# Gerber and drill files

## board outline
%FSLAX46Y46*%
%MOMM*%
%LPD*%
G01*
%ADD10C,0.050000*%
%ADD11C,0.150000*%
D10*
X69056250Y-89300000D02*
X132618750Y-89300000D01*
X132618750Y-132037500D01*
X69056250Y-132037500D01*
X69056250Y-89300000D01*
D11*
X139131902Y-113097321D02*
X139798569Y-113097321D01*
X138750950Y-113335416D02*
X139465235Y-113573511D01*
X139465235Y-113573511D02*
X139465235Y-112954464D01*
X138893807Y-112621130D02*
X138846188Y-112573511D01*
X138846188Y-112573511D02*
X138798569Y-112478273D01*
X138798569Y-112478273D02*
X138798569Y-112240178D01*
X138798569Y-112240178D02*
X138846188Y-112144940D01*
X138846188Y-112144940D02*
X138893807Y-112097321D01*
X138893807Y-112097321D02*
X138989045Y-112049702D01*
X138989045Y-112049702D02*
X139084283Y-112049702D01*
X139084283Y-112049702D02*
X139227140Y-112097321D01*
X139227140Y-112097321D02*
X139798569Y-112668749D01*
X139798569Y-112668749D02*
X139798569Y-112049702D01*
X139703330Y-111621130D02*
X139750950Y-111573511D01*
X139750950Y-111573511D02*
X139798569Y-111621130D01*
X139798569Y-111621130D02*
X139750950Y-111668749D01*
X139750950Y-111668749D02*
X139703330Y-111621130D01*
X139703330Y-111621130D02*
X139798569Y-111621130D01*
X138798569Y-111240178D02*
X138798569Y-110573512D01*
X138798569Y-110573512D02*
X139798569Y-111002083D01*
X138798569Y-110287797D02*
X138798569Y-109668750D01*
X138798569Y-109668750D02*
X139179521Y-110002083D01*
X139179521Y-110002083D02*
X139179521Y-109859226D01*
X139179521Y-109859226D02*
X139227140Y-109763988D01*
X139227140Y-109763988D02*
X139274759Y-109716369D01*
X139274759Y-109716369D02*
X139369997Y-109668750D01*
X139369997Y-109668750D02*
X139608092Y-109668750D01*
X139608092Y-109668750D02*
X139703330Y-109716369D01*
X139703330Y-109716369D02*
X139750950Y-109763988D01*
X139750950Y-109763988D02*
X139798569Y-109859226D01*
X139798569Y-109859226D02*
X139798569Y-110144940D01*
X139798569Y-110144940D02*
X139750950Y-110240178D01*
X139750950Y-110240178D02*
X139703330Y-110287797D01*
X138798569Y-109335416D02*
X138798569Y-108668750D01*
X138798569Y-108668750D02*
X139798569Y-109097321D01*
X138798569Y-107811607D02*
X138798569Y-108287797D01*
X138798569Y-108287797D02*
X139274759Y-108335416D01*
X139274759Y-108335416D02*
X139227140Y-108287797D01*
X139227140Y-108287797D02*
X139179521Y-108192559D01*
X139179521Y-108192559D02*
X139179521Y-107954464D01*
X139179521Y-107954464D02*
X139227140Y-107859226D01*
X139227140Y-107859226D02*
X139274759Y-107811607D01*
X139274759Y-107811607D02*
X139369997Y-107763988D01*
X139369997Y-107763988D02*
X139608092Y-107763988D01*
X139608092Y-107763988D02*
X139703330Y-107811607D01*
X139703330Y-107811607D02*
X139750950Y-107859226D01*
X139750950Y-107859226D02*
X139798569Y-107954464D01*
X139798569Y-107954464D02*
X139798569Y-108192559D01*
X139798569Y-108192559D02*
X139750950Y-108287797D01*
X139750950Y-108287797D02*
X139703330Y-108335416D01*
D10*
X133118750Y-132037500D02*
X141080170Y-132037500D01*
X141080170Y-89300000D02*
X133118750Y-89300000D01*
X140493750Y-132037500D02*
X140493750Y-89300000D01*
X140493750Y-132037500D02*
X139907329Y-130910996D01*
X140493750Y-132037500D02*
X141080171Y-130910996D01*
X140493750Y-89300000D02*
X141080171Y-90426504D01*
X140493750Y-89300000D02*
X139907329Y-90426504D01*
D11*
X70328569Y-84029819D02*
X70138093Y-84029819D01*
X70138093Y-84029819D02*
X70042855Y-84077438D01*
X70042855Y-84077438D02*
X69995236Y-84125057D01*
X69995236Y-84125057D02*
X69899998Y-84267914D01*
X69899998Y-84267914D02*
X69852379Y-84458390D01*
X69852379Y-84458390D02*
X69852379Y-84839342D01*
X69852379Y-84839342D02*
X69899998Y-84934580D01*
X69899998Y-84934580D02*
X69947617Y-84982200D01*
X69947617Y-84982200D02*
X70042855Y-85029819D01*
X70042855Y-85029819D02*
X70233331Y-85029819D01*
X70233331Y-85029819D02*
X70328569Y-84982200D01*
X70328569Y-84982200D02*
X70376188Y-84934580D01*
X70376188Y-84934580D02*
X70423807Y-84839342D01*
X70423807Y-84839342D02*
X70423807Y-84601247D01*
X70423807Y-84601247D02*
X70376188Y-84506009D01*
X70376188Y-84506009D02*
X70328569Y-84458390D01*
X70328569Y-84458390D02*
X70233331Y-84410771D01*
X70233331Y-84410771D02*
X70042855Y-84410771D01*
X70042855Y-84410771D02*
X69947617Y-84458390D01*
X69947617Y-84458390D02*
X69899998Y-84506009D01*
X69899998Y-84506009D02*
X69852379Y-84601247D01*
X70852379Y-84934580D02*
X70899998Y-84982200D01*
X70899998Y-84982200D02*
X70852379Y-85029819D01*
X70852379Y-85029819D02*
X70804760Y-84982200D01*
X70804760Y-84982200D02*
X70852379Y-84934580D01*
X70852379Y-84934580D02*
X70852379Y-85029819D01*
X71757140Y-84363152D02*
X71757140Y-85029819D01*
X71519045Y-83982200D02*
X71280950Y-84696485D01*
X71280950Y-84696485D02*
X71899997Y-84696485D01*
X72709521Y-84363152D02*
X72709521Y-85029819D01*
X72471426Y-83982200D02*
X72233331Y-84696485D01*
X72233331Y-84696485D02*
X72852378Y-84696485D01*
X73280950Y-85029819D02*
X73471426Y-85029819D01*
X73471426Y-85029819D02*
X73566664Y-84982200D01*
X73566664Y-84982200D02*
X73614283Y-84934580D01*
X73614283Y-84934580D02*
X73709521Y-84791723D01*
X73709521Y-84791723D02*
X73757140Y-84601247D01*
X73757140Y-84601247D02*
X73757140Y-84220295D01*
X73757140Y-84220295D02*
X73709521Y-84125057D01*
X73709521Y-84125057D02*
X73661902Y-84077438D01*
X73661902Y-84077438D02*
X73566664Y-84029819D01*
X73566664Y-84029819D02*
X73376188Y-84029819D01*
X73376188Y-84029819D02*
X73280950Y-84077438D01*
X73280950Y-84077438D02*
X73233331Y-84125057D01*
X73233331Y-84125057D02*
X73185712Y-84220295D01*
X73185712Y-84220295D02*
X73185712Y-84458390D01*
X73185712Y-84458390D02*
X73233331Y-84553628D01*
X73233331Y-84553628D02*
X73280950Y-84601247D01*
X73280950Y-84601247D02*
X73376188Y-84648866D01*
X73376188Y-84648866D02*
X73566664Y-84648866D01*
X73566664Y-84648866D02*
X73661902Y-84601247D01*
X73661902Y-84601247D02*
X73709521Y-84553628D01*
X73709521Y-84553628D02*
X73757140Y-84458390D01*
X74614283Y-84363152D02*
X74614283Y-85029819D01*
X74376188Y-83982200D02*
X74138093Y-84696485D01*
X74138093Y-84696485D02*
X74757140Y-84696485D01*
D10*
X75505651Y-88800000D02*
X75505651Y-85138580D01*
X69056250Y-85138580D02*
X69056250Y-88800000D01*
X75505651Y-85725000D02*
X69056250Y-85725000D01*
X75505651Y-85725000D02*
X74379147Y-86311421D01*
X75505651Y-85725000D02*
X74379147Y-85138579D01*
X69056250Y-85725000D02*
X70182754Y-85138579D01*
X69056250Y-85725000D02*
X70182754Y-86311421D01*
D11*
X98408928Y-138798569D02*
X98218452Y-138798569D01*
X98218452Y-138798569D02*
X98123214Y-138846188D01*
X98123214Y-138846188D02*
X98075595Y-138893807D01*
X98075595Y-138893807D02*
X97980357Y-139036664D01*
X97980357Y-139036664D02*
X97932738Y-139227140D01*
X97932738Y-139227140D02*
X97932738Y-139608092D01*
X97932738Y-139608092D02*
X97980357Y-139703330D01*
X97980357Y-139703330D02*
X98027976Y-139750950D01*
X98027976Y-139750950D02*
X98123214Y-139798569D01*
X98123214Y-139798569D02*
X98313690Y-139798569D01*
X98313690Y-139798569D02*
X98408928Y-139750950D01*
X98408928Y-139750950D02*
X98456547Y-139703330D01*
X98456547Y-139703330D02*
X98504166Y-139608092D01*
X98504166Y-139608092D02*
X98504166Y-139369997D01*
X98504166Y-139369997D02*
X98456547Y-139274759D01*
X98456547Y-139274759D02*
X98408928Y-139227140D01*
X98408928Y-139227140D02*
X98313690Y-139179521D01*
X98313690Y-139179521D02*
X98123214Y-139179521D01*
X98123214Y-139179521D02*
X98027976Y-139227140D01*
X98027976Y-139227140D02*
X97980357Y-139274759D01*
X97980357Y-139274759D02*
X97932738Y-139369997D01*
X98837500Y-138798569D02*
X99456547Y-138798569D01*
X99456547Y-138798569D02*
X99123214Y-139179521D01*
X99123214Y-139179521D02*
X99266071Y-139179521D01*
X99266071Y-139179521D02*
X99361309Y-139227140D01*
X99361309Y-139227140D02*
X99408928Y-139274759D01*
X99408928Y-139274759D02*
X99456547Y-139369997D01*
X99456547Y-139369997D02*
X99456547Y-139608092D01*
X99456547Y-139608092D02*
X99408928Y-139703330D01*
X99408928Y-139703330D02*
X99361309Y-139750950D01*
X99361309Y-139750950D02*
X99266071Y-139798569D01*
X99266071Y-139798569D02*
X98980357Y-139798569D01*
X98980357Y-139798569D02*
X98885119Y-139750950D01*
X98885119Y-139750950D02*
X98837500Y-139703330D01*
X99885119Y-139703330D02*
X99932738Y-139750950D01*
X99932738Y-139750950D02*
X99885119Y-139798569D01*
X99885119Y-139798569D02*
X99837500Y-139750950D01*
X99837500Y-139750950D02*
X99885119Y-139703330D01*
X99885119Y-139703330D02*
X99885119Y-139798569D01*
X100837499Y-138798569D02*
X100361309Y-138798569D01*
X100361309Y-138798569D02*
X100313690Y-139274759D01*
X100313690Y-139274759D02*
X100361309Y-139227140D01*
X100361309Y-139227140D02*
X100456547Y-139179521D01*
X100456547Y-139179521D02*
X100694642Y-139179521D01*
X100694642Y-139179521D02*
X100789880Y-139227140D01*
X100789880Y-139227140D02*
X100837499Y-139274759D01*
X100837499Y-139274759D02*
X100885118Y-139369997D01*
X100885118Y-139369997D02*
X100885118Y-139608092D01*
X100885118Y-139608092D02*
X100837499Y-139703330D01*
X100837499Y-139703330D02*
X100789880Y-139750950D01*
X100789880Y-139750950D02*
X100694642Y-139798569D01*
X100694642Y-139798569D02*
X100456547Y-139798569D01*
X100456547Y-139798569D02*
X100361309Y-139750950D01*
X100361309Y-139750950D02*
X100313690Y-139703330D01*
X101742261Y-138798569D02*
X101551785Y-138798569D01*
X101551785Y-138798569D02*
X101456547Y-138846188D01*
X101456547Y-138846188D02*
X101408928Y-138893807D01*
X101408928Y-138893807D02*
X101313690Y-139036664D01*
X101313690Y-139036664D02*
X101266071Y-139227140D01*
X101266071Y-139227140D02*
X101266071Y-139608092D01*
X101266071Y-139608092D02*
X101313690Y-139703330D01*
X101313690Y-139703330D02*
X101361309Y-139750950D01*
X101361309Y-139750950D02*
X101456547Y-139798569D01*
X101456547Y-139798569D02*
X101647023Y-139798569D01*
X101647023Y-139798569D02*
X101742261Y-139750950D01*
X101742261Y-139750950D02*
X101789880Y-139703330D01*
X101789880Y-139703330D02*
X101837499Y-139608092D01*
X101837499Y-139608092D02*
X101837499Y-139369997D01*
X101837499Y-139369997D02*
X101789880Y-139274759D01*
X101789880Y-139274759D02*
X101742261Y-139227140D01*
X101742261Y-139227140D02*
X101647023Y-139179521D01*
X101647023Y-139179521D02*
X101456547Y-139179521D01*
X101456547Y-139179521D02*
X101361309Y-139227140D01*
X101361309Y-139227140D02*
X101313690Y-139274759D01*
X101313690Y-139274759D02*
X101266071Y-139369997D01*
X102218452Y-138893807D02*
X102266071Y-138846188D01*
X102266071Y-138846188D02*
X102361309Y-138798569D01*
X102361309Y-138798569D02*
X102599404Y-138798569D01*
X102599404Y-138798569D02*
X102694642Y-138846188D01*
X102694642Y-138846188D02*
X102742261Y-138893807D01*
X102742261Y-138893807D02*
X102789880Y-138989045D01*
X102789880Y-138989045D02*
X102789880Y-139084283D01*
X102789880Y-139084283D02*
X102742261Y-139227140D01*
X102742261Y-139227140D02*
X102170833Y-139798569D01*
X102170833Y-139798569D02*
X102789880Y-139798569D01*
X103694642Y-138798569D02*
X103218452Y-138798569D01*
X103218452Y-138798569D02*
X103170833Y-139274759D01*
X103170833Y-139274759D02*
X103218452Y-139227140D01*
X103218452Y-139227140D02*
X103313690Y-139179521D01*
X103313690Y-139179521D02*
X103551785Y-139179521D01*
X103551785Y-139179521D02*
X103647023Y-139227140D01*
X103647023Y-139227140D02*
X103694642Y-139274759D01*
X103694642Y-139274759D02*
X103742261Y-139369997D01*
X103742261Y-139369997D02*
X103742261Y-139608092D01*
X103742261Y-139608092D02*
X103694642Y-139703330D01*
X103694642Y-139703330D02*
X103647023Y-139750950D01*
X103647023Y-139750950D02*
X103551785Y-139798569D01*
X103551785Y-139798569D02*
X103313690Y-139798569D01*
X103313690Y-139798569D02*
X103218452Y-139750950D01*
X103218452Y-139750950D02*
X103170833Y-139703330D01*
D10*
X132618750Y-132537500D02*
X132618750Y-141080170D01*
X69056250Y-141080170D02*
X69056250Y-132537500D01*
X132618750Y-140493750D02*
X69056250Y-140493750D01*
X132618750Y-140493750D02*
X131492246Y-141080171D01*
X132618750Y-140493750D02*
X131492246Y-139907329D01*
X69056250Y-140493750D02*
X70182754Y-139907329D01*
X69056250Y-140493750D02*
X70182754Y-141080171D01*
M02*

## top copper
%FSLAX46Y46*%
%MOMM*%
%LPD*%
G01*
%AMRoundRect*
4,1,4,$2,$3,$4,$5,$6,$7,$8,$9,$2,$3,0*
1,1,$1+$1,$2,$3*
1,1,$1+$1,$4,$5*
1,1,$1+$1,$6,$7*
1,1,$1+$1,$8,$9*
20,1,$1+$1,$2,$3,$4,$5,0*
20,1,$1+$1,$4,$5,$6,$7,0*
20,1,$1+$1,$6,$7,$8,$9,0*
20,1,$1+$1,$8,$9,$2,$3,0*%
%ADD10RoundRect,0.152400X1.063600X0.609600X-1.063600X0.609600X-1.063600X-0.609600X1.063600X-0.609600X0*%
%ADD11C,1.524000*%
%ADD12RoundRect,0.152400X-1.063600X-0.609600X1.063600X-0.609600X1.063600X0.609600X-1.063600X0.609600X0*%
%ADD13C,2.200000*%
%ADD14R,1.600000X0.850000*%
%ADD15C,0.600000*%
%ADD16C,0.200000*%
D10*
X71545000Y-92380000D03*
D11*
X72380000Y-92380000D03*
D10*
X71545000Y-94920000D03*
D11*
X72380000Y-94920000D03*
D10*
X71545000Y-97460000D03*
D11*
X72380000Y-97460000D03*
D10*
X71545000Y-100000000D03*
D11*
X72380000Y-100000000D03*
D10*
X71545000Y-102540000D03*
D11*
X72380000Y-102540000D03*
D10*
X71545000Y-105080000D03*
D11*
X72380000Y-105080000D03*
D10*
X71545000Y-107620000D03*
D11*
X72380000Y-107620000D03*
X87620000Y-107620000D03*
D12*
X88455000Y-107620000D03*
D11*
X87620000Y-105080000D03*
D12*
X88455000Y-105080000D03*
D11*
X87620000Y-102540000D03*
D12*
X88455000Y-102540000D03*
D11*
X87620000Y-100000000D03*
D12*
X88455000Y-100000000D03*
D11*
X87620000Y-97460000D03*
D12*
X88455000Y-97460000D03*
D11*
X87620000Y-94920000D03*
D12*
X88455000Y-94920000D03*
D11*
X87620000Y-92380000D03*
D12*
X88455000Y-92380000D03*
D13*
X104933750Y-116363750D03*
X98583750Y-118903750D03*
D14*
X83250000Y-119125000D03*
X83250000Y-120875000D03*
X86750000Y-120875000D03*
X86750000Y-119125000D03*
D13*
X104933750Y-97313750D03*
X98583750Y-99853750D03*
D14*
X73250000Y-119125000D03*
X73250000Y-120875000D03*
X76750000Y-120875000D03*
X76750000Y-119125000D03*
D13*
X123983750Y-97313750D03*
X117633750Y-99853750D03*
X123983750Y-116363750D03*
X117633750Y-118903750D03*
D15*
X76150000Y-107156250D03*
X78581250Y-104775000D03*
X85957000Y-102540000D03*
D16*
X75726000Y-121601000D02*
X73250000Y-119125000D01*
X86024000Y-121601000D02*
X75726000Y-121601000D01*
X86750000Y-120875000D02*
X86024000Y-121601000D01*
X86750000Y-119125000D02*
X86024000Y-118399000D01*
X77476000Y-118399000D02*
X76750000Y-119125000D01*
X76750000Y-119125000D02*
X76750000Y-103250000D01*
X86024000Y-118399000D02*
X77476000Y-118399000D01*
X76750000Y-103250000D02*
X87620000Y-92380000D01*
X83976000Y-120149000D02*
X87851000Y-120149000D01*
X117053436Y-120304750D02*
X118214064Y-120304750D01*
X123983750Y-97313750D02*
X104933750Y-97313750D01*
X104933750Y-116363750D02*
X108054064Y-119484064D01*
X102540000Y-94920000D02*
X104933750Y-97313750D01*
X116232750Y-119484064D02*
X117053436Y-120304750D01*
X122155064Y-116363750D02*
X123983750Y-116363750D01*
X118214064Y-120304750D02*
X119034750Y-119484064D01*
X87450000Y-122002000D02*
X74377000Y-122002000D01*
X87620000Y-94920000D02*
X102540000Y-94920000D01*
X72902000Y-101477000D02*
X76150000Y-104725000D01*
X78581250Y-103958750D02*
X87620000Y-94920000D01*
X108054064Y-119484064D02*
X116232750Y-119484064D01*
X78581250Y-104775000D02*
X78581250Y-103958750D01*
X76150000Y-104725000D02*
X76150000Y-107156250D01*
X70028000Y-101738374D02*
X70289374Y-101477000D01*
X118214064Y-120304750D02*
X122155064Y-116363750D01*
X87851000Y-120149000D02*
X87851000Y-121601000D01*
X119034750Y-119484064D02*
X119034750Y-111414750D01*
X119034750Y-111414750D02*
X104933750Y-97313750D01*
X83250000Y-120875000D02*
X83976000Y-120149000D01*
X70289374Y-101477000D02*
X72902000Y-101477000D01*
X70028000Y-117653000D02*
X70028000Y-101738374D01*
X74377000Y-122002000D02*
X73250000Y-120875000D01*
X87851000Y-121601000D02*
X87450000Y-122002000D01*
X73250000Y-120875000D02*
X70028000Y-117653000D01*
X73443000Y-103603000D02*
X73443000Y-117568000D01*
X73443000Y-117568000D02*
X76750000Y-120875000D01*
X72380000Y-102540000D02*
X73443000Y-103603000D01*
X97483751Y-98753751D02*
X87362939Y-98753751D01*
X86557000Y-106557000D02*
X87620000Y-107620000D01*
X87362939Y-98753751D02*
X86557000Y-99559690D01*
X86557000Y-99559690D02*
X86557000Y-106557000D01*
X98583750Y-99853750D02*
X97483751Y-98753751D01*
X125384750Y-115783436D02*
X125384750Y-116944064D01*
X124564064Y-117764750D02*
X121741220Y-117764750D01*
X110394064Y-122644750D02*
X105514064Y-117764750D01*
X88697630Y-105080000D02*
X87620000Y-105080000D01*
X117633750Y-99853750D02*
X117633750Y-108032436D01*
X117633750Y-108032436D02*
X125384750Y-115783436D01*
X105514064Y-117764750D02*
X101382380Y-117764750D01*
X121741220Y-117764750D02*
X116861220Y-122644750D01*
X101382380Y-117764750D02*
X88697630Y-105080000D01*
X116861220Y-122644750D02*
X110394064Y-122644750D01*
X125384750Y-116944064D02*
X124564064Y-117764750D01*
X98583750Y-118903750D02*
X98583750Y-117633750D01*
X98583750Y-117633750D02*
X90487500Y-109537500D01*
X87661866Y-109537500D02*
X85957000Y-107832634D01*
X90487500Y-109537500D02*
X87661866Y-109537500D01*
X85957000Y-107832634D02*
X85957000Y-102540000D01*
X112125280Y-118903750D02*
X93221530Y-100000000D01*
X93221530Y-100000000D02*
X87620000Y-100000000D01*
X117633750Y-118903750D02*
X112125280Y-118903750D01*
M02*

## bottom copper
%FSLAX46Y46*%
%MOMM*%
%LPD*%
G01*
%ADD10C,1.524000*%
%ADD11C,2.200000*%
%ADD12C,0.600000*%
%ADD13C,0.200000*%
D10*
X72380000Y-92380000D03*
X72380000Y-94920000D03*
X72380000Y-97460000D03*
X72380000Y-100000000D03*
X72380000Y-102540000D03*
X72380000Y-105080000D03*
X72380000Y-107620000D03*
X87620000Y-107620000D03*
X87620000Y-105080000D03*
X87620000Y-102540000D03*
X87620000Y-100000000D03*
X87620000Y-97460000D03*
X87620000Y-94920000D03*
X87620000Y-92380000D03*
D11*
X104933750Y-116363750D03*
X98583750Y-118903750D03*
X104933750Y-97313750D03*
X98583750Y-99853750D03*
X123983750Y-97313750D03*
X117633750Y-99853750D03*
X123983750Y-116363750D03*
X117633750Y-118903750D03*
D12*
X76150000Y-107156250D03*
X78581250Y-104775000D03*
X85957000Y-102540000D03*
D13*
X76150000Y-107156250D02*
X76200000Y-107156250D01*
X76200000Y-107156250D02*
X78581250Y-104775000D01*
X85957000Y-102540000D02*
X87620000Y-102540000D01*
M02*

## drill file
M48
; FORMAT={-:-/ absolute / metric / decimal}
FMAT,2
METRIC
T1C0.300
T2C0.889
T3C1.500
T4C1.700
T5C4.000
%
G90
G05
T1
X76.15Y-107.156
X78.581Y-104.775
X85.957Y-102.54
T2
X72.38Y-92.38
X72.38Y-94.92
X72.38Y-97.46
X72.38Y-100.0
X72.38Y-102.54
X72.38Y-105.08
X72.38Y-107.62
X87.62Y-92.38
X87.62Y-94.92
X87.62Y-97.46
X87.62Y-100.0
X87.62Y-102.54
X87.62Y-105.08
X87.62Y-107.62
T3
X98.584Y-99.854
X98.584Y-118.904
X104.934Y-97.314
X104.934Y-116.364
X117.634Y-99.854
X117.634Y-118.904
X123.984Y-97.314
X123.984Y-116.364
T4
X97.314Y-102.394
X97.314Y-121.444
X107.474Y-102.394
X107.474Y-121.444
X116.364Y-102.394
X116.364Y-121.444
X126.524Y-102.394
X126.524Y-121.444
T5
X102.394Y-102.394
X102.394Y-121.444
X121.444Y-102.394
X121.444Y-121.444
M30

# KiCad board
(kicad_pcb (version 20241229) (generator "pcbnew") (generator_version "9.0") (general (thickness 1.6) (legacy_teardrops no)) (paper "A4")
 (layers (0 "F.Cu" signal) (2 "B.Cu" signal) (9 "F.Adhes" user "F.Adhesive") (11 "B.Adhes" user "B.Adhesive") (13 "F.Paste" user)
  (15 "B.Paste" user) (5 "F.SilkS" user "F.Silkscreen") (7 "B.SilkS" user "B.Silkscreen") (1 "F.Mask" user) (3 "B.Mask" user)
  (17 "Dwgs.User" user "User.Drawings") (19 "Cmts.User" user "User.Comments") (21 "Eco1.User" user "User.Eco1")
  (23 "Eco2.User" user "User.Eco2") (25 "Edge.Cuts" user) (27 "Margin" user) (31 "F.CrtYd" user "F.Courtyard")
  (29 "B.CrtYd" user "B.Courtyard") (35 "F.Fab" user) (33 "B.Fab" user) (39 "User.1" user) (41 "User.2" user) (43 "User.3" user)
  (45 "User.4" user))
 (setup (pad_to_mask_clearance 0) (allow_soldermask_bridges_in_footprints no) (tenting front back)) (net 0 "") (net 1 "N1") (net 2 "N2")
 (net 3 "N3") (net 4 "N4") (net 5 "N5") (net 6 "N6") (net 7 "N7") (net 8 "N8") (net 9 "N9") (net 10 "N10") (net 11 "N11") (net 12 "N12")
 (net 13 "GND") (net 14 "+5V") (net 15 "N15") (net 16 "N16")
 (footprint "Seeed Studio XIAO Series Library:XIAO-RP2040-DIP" (layer "F.Cu") (at 80 100)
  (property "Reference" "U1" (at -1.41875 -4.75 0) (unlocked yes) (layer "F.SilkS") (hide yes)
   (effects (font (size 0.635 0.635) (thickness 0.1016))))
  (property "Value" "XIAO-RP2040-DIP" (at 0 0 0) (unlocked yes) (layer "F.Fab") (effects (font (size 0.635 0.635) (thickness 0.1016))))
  (pad "1" smd roundrect (at -8.455 -7.62 180) (size 2.432 1.524) (layers "F.Cu" "F.Mask") (roundrect_rratio 0.1) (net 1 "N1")
   (thermal_bridge_angle 45))
  (pad "1" thru_hole circle (at -7.62 -7.62 180) (size 1.524 1.524) (drill 0.889) (layers "*.Cu" "*.Mask") (remove_unused_layers no)
   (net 1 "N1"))
  (pad "2" smd roundrect (at -8.455 -5.08 180) (size 2.432 1.524) (layers "F.Cu" "F.Mask") (roundrect_rratio 0.1) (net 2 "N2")
   (thermal_bridge_angle 45))
  (pad "2" thru_hole circle (at -7.62 -5.08 180) (size 1.524 1.524) (drill 0.889) (layers "*.Cu" "*.Mask") (remove_unused_layers no)
   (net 2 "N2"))
  (pad "3" smd roundrect (at -8.455 -2.54 180) (size 2.432 1.524) (layers "F.Cu" "F.Mask") (roundrect_rratio 0.1) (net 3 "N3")
   (thermal_bridge_angle 45))
  (pad "3" thru_hole circle (at -7.62 -2.54 180) (size 1.524 1.524) (drill 0.889) (layers "*.Cu" "*.Mask") (remove_unused_layers no)
   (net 3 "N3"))
  (pad "4" smd roundrect (at -8.455 0 180) (size 2.432 1.524) (layers "F.Cu" "F.Mask") (roundrect_rratio 0.1) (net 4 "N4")
   (thermal_bridge_angle 45))
  (pad "4" thru_hole circle (at -7.62 0 180) (size 1.524 1.524) (drill 0.889) (layers "*.Cu" "*.Mask") (remove_unused_layers no)
   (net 4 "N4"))
  (pad "5" smd roundrect (at -8.455 2.54 180) (size 2.432 1.524) (layers "F.Cu" "F.Mask") (roundrect_rratio 0.1) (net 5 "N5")
   (thermal_bridge_angle 45))
  (pad "5" thru_hole circle (at -7.62 2.54 180) (size 1.524 1.524) (drill 0.889) (layers "*.Cu" "*.Mask") (remove_unused_layers no)
   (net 5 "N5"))
  (pad "6" smd roundrect (at -8.455 5.08 180) (size 2.432 1.524) (layers "F.Cu" "F.Mask") (roundrect_rratio 0.1) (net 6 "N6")
   (thermal_bridge_angle 45))
  (pad "6" thru_hole circle (at -7.62 5.08 180) (size 1.524 1.524) (drill 0.889) (layers "*.Cu" "*.Mask") (remove_unused_layers no)
   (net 6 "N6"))
  (pad "7" smd roundrect (at -8.455 7.62 180) (size 2.432 1.524) (layers "F.Cu" "F.Mask") (roundrect_rratio 0.1) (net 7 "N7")
   (thermal_bridge_angle 45))
  (pad "7" thru_hole circle (at -7.62 7.62 180) (size 1.524 1.524) (drill 0.889) (layers "*.Cu" "*.Mask") (remove_unused_layers no)
   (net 7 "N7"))
  (pad "8" thru_hole circle (at 7.62 7.62) (size 1.524 1.524) (drill 0.889) (layers "*.Cu" "*.Mask") (remove_unused_layers no) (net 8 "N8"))
  (pad "8" smd roundrect (at 8.455 7.62) (size 2.432 1.524) (layers "F.Cu" "F.Mask") (roundrect_rratio 0.1) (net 8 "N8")
   (thermal_bridge_angle 45))
  (pad "9" thru_hole circle (at 7.62 5.08) (size 1.524 1.524) (drill 0.889) (layers "*.Cu" "*.Mask") (remove_unused_layers no) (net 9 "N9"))
  (pad "9" smd roundrect (at 8.455 5.08) (size 2.432 1.524) (layers "F.Cu" "F.Mask") (roundrect_rratio 0.1) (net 9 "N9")
   (thermal_bridge_angle 45))
  (pad "10" thru_hole circle (at 7.62 2.54) (size 1.524 1.524) (drill 0.889) (layers "*.Cu" "*.Mask") (remove_unused_layers no)
   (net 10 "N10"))
  (pad "10" smd roundrect (at 8.455 2.54) (size 2.432 1.524) (layers "F.Cu" "F.Mask") (roundrect_rratio 0.1) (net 10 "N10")
   (thermal_bridge_angle 45))
  (pad "11" thru_hole circle (at 7.62 0) (size 1.524 1.524) (drill 0.889) (layers "*.Cu" "*.Mask") (remove_unused_layers no) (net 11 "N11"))
  (pad "11" smd roundrect (at 8.455 0) (size 2.432 1.524) (layers "F.Cu" "F.Mask") (roundrect_rratio 0.1) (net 11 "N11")
   (thermal_bridge_angle 45))
  (pad "12" thru_hole circle (at 7.62 -2.54) (size 1.524 1.524) (drill 0.889) (layers "*.Cu" "*.Mask") (remove_unused_layers no)
   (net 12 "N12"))
  (pad "12" smd roundrect (at 8.455 -2.54) (size 2.432 1.524) (layers "F.Cu" "F.Mask") (roundrect_rratio 0.1) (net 12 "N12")
   (thermal_bridge_angle 45))
  (pad "13" thru_hole circle (at 7.62 -5.08) (size 1.524 1.524) (drill 0.889) (layers "*.Cu" "*.Mask") (remove_unused_layers no)
   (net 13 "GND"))
  (pad "13" smd roundrect (at 8.455 -5.08) (size 2.432 1.524) (layers "F.Cu" "F.Mask") (roundrect_rratio 0.1) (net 13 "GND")
   (thermal_bridge_angle 45))
  (pad "14" thru_hole circle (at 7.62 -7.62) (size 1.524 1.524) (drill 0.889) (layers "*.Cu" "*.Mask") (remove_unused_layers no)
   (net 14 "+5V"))
  (pad "14" smd roundrect (at 8.455 -7.62) (size 2.432 1.524) (layers "F.Cu" "F.Mask") (roundrect_rratio 0.1) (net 14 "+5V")
   (thermal_bridge_angle 45)))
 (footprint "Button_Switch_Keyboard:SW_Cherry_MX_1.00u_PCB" (layer "F.Cu") (at 104.93375 116.36375)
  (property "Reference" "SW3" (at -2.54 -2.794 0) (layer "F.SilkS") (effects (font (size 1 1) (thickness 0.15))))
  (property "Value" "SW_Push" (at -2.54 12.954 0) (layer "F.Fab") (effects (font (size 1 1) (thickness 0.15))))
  (pad "" np_thru_hole circle (at -7.62 5.08) (size 1.7 1.7) (drill 1.7) (layers "*.Cu" "*.Mask"))
  (pad "" np_thru_hole circle (at -2.54 5.08) (size 4 4) (drill 4) (layers "*.Cu" "*.Mask"))
  (pad "" np_thru_hole circle (at 2.54 5.08) (size 1.7 1.7) (drill 1.7) (layers "*.Cu" "*.Mask"))
  (pad "1" thru_hole circle (at 0 0) (size 2.2 2.2) (drill 1.5) (layers "*.Cu" "*.Mask") (remove_unused_layers no) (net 13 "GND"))
  (pad "2" thru_hole circle (at -6.35 2.54) (size 2.2 2.2) (drill 1.5) (layers "*.Cu" "*.Mask") (remove_unused_layers no) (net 10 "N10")))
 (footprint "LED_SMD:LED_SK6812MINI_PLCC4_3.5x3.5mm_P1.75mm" (layer "F.Cu") (at 85 120)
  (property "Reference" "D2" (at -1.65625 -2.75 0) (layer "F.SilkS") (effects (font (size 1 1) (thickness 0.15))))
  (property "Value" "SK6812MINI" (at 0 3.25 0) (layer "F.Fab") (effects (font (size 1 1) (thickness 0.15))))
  (pad "1" smd rect (at -1.75 -0.875) (size 1.6 0.85) (layers "F.Cu" "F.Mask" "F.Paste") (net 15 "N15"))
  (pad "2" smd rect (at -1.75 0.875) (size 1.6 0.85) (layers "F.Cu" "F.Mask" "F.Paste") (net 13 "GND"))
  (pad "3" smd rect (at 1.75 0.875) (size 1.6 0.85) (layers "F.Cu" "F.Mask" "F.Paste") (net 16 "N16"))
  (pad "4" smd rect (at 1.75 -0.875) (size 1.6 0.85) (layers "F.Cu" "F.Mask" "F.Paste") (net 14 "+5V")))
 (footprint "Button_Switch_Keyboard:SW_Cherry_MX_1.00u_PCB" (layer "F.Cu") (at 104.93375 97.31375)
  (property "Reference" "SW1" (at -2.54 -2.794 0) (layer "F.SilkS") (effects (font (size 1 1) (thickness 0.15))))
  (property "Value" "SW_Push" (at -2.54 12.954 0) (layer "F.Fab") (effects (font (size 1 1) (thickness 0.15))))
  (pad "" np_thru_hole circle (at -7.62 5.08) (size 1.7 1.7) (drill 1.7) (layers "*.Cu" "*.Mask"))
  (pad "" np_thru_hole circle (at -2.54 5.08) (size 4 4) (drill 4) (layers "*.Cu" "*.Mask"))
  (pad "" np_thru_hole circle (at 2.54 5.08) (size 1.7 1.7) (drill 1.7) (layers "*.Cu" "*.Mask"))
  (pad "1" thru_hole circle (at 0 0) (size 2.2 2.2) (drill 1.5) (layers "*.Cu" "*.Mask") (remove_unused_layers no) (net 13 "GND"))
  (pad "2" thru_hole circle (at -6.35 2.54) (size 2.2 2.2) (drill 1.5) (layers "*.Cu" "*.Mask") (remove_unused_layers no) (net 8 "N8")))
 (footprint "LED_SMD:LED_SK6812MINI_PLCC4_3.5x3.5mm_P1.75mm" (layer "F.Cu") (at 75 120)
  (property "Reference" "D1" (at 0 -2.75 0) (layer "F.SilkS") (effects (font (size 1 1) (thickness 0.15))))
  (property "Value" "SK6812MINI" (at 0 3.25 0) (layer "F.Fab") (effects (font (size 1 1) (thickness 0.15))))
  (pad "1" smd rect (at -1.75 -0.875) (size 1.6 0.85) (layers "F.Cu" "F.Mask" "F.Paste") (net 16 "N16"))
  (pad "2" smd rect (at -1.75 0.875) (size 1.6 0.85) (layers "F.Cu" "F.Mask" "F.Paste") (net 13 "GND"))
  (pad "3" smd rect (at 1.75 0.875) (size 1.6 0.85) (layers "F.Cu" "F.Mask" "F.Paste") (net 5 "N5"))
  (pad "4" smd rect (at 1.75 -0.875) (size 1.6 0.85) (layers "F.Cu" "F.Mask" "F.Paste") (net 14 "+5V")))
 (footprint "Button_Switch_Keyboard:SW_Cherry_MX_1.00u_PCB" (layer "F.Cu") (at 123.98375 97.31375)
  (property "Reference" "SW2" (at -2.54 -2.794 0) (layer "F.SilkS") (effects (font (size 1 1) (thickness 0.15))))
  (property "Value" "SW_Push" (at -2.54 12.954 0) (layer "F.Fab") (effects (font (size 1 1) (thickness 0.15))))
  (pad "" np_thru_hole circle (at -7.62 5.08) (size 1.7 1.7) (drill 1.7) (layers "*.Cu" "*.Mask"))
  (pad "" np_thru_hole circle (at -2.54 5.08) (size 4 4) (drill 4) (layers "*.Cu" "*.Mask"))
  (pad "" np_thru_hole circle (at 2.54 5.08) (size 1.7 1.7) (drill 1.7) (layers "*.Cu" "*.Mask"))
  (pad "1" thru_hole circle (at 0 0) (size 2.2 2.2) (drill 1.5) (layers "*.Cu" "*.Mask") (remove_unused_layers no) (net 13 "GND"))
  (pad "2" thru_hole circle (at -6.35 2.54) (size 2.2 2.2) (drill 1.5) (layers "*.Cu" "*.Mask") (remove_unused_layers no) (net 9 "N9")))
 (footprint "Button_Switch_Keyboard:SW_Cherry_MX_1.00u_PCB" (layer "F.Cu") (at 123.98375 116.36375)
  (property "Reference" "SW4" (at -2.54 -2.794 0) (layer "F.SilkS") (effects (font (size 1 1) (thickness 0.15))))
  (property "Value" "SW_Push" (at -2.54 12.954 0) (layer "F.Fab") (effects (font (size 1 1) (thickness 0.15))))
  (pad "" np_thru_hole circle (at -7.62 5.08) (size 1.7 1.7) (drill 1.7) (layers "*.Cu" "*.Mask"))
  (pad "" np_thru_hole circle (at -2.54 5.08) (size 4 4) (drill 4) (layers "*.Cu" "*.Mask"))
  (pad "" np_thru_hole circle (at 2.54 5.08) (size 1.7 1.7) (drill 1.7) (layers "*.Cu" "*.Mask"))
  (pad "1" thru_hole circle (at 0 0) (size 2.2 2.2) (drill 1.5) (layers "*.Cu" "*.Mask") (remove_unused_layers no) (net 13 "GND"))
  (pad "2" thru_hole circle (at -6.35 2.54) (size 2.2 2.2) (drill 1.5) (layers "*.Cu" "*.Mask") (remove_unused_layers no) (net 11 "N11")))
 (gr_rect (start 69.05625 89.3) (end 132.61875 132.0375) (stroke (width 0.05) (type solid)) (fill no) (layer "Edge.Cuts"))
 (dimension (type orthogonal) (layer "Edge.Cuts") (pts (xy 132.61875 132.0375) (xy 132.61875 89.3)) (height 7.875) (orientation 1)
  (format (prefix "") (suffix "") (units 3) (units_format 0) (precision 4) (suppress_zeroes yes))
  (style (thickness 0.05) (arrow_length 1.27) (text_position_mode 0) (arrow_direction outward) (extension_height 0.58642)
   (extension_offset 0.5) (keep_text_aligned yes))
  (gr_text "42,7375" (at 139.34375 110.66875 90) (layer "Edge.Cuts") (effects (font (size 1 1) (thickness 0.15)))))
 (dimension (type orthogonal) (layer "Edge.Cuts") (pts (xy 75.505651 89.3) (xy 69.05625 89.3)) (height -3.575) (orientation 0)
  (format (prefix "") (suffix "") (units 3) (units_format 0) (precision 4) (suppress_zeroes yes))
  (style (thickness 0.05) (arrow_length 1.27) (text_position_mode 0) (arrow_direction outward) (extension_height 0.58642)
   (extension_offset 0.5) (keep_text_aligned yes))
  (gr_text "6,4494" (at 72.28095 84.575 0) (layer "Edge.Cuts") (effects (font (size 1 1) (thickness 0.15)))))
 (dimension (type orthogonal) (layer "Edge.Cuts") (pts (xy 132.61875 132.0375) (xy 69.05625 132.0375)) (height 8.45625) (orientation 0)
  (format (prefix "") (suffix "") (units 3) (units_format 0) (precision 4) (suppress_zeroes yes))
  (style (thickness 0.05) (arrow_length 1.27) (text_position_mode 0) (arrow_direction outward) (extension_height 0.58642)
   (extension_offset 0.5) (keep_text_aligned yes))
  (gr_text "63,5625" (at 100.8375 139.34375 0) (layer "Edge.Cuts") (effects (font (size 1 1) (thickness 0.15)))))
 (segment (start 75.726 121.601) (end 73.25 119.125) (width 0.2) (layer "F.Cu") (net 16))
 (segment (start 86.024 121.601) (end 75.726 121.601) (width 0.2) (layer "F.Cu") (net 16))
 (segment (start 86.75 120.875) (end 86.024 121.601) (width 0.2) (layer "F.Cu") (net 16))
 (segment (start 86.75 119.125) (end 86.024 118.399) (width 0.2) (layer "F.Cu") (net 14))
 (segment (start 77.476 118.399) (end 76.75 119.125) (width 0.2) (layer "F.Cu") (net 14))
 (segment (start 76.75 119.125) (end 76.75 103.25) (width 0.2) (layer "F.Cu") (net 14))
 (segment (start 86.024 118.399) (end 77.476 118.399) (width 0.2) (layer "F.Cu") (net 14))
 (segment (start 76.75 103.25) (end 87.62 92.38) (width 0.2) (layer "F.Cu") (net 14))
 (segment (start 83.976 120.149) (end 87.851 120.149) (width 0.2) (layer "F.Cu") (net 13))
 (segment (start 117.053436 120.30475) (end 118.214064 120.30475) (width 0.2) (layer "F.Cu") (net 13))
 (segment (start 123.98375 97.31375) (end 104.93375 97.31375) (width 0.2) (layer "F.Cu") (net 13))
 (segment (start 104.93375 116.36375) (end 108.054064 119.484064) (width 0.2) (layer "F.Cu") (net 13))
 (segment (start 102.54 94.92) (end 104.93375 97.31375) (width 0.2) (layer "F.Cu") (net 13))
 (segment (start 116.23275 119.484064) (end 117.053436 120.30475) (width 0.2) (layer "F.Cu") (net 13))
 (segment (start 122.155064 116.36375) (end 123.98375 116.36375) (width 0.2) (layer "F.Cu") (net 13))
 (segment (start 118.214064 120.30475) (end 119.03475 119.484064) (width 0.2) (layer "F.Cu") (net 13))
 (segment (start 87.45 122.002) (end 74.377 122.002) (width 0.2) (layer "F.Cu") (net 13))
 (segment (start 87.62 94.92) (end 102.54 94.92) (width 0.2) (layer "F.Cu") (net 13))
 (segment (start 72.902 101.477) (end 76.15 104.725) (width 0.2) (layer "F.Cu") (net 13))
 (segment (start 78.58125 103.95875) (end 87.62 94.92) (width 0.2) (layer "F.Cu") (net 13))
 (segment (start 108.054064 119.484064) (end 116.23275 119.484064) (width 0.2) (layer "F.Cu") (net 13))
 (segment (start 78.58125 104.775) (end 78.58125 103.95875) (width 0.2) (layer "F.Cu") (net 13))
 (segment (start 76.15 104.725) (end 76.15 107.15625) (width 0.2) (layer "F.Cu") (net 13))
 (segment (start 70.028 101.738374) (end 70.289374 101.477) (width 0.2) (layer "F.Cu") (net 13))
 (segment (start 118.214064 120.30475) (end 122.155064 116.36375) (width 0.2) (layer "F.Cu") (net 13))
 (segment (start 87.851 120.149) (end 87.851 121.601) (width 0.2) (layer "F.Cu") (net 13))
 (segment (start 119.03475 119.484064) (end 119.03475 111.41475) (width 0.2) (layer "F.Cu") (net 13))
 (segment (start 119.03475 111.41475) (end 104.93375 97.31375) (width 0.2) (layer "F.Cu") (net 13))
 (segment (start 83.25 120.875) (end 83.976 120.149) (width 0.2) (layer "F.Cu") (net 13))
 (segment (start 70.289374 101.477) (end 72.902 101.477) (width 0.2) (layer "F.Cu") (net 13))
 (segment (start 70.028 117.653) (end 70.028 101.738374) (width 0.2) (layer "F.Cu") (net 13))
 (segment (start 74.377 122.002) (end 73.25 120.875) (width 0.2) (layer "F.Cu") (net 13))
 (segment (start 87.851 121.601) (end 87.45 122.002) (width 0.2) (layer "F.Cu") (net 13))
 (segment (start 73.25 120.875) (end 70.028 117.653) (width 0.2) (layer "F.Cu") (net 13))
 (via (at 76.15 107.15625) (size 0.6) (drill 0.3) (layers "F.Cu" "B.Cu") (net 13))
 (via (at 78.58125 104.775) (size 0.6) (drill 0.3) (layers "F.Cu" "B.Cu") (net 13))
 (segment (start 76.15 107.15625) (end 76.2 107.15625) (width 0.2) (layer "B.Cu") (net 13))
 (segment (start 76.2 107.15625) (end 78.58125 104.775) (width 0.2) (layer "B.Cu") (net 13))
 (segment (start 73.443 103.603) (end 73.443 117.568) (width 0.2) (layer "F.Cu") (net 5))
 (segment (start 73.443 117.568) (end 76.75 120.875) (width 0.2) (layer "F.Cu") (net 5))
 (segment (start 72.38 102.54) (end 73.443 103.603) (width 0.2) (layer "F.Cu") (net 5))
 (segment (start 97.483751 98.753751) (end 87.362939 98.753751) (width 0.2) (layer "F.Cu") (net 8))
 (segment (start 86.557 106.557) (end 87.62 107.62) (width 0.2) (layer "F.Cu") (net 8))
 (segment (start 87.362939 98.753751) (end 86.557 99.55969) (width 0.2) (layer "F.Cu") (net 8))
 (segment (start 86.557 99.55969) (end 86.557 106.557) (width 0.2) (layer "F.Cu") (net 8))
 (segment (start 98.58375 99.85375) (end 97.483751 98.753751) (width 0.2) (layer "F.Cu") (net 8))
 (segment (start 125.38475 115.783436) (end 125.38475 116.944064) (width 0.2) (layer "F.Cu") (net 9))
 (segment (start 124.564064 117.76475) (end 121.74122 117.76475) (width 0.2) (layer "F.Cu") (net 9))
 (segment (start 110.394064 122.64475) (end 105.514064 117.76475) (width 0.2) (layer "F.Cu") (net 9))
 (segment (start 88.69763 105.08) (end 87.62 105.08) (width 0.2) (layer "F.Cu") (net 9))
 (segment (start 117.63375 99.85375) (end 117.63375 108.032436) (width 0.2) (layer "F.Cu") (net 9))
 (segment (start 117.63375 108.032436) (end 125.38475 115.783436) (width 0.2) (layer "F.Cu") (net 9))
 (segment (start 105.514064 117.76475) (end 101.38238 117.76475) (width 0.2) (layer "F.Cu") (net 9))
 (segment (start 121.74122 117.76475) (end 116.86122 122.64475) (width 0.2) (layer "F.Cu") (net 9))
 (segment (start 101.38238 117.76475) (end 88.69763 105.08) (width 0.2) (layer "F.Cu") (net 9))
 (segment (start 116.86122 122.64475) (end 110.394064 122.64475) (width 0.2) (layer "F.Cu") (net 9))
 (segment (start 125.38475 116.944064) (end 124.564064 117.76475) (width 0.2) (layer "F.Cu") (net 9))
 (segment (start 98.58375 118.90375) (end 98.58375 117.63375) (width 0.2) (layer "F.Cu") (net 10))
 (segment (start 98.58375 117.63375) (end 90.4875 109.5375) (width 0.2) (layer "F.Cu") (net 10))
 (segment (start 87.661866 109.5375) (end 85.957 107.832634) (width 0.2) (layer "F.Cu") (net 10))
 (segment (start 90.4875 109.5375) (end 87.661866 109.5375) (width 0.2) (layer "F.Cu") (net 10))
 (segment (start 85.957 107.832634) (end 85.957 102.54) (width 0.2) (layer "F.Cu") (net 10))
 (via (at 85.957 102.54) (size 0.6) (drill 0.3) (layers "F.Cu" "B.Cu") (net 10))
 (segment (start 85.957 102.54) (end 87.62 102.54) (width 0.2) (layer "B.Cu") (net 10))
 (segment (start 112.12528 118.90375) (end 93.22153 100) (width 0.2) (layer "F.Cu") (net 11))
 (segment (start 93.22153 100) (end 87.62 100) (width 0.2) (layer "F.Cu") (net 11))
 (segment (start 117.63375 118.90375) (end 112.12528 118.90375) (width 0.2) (layer "F.Cu") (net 11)))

